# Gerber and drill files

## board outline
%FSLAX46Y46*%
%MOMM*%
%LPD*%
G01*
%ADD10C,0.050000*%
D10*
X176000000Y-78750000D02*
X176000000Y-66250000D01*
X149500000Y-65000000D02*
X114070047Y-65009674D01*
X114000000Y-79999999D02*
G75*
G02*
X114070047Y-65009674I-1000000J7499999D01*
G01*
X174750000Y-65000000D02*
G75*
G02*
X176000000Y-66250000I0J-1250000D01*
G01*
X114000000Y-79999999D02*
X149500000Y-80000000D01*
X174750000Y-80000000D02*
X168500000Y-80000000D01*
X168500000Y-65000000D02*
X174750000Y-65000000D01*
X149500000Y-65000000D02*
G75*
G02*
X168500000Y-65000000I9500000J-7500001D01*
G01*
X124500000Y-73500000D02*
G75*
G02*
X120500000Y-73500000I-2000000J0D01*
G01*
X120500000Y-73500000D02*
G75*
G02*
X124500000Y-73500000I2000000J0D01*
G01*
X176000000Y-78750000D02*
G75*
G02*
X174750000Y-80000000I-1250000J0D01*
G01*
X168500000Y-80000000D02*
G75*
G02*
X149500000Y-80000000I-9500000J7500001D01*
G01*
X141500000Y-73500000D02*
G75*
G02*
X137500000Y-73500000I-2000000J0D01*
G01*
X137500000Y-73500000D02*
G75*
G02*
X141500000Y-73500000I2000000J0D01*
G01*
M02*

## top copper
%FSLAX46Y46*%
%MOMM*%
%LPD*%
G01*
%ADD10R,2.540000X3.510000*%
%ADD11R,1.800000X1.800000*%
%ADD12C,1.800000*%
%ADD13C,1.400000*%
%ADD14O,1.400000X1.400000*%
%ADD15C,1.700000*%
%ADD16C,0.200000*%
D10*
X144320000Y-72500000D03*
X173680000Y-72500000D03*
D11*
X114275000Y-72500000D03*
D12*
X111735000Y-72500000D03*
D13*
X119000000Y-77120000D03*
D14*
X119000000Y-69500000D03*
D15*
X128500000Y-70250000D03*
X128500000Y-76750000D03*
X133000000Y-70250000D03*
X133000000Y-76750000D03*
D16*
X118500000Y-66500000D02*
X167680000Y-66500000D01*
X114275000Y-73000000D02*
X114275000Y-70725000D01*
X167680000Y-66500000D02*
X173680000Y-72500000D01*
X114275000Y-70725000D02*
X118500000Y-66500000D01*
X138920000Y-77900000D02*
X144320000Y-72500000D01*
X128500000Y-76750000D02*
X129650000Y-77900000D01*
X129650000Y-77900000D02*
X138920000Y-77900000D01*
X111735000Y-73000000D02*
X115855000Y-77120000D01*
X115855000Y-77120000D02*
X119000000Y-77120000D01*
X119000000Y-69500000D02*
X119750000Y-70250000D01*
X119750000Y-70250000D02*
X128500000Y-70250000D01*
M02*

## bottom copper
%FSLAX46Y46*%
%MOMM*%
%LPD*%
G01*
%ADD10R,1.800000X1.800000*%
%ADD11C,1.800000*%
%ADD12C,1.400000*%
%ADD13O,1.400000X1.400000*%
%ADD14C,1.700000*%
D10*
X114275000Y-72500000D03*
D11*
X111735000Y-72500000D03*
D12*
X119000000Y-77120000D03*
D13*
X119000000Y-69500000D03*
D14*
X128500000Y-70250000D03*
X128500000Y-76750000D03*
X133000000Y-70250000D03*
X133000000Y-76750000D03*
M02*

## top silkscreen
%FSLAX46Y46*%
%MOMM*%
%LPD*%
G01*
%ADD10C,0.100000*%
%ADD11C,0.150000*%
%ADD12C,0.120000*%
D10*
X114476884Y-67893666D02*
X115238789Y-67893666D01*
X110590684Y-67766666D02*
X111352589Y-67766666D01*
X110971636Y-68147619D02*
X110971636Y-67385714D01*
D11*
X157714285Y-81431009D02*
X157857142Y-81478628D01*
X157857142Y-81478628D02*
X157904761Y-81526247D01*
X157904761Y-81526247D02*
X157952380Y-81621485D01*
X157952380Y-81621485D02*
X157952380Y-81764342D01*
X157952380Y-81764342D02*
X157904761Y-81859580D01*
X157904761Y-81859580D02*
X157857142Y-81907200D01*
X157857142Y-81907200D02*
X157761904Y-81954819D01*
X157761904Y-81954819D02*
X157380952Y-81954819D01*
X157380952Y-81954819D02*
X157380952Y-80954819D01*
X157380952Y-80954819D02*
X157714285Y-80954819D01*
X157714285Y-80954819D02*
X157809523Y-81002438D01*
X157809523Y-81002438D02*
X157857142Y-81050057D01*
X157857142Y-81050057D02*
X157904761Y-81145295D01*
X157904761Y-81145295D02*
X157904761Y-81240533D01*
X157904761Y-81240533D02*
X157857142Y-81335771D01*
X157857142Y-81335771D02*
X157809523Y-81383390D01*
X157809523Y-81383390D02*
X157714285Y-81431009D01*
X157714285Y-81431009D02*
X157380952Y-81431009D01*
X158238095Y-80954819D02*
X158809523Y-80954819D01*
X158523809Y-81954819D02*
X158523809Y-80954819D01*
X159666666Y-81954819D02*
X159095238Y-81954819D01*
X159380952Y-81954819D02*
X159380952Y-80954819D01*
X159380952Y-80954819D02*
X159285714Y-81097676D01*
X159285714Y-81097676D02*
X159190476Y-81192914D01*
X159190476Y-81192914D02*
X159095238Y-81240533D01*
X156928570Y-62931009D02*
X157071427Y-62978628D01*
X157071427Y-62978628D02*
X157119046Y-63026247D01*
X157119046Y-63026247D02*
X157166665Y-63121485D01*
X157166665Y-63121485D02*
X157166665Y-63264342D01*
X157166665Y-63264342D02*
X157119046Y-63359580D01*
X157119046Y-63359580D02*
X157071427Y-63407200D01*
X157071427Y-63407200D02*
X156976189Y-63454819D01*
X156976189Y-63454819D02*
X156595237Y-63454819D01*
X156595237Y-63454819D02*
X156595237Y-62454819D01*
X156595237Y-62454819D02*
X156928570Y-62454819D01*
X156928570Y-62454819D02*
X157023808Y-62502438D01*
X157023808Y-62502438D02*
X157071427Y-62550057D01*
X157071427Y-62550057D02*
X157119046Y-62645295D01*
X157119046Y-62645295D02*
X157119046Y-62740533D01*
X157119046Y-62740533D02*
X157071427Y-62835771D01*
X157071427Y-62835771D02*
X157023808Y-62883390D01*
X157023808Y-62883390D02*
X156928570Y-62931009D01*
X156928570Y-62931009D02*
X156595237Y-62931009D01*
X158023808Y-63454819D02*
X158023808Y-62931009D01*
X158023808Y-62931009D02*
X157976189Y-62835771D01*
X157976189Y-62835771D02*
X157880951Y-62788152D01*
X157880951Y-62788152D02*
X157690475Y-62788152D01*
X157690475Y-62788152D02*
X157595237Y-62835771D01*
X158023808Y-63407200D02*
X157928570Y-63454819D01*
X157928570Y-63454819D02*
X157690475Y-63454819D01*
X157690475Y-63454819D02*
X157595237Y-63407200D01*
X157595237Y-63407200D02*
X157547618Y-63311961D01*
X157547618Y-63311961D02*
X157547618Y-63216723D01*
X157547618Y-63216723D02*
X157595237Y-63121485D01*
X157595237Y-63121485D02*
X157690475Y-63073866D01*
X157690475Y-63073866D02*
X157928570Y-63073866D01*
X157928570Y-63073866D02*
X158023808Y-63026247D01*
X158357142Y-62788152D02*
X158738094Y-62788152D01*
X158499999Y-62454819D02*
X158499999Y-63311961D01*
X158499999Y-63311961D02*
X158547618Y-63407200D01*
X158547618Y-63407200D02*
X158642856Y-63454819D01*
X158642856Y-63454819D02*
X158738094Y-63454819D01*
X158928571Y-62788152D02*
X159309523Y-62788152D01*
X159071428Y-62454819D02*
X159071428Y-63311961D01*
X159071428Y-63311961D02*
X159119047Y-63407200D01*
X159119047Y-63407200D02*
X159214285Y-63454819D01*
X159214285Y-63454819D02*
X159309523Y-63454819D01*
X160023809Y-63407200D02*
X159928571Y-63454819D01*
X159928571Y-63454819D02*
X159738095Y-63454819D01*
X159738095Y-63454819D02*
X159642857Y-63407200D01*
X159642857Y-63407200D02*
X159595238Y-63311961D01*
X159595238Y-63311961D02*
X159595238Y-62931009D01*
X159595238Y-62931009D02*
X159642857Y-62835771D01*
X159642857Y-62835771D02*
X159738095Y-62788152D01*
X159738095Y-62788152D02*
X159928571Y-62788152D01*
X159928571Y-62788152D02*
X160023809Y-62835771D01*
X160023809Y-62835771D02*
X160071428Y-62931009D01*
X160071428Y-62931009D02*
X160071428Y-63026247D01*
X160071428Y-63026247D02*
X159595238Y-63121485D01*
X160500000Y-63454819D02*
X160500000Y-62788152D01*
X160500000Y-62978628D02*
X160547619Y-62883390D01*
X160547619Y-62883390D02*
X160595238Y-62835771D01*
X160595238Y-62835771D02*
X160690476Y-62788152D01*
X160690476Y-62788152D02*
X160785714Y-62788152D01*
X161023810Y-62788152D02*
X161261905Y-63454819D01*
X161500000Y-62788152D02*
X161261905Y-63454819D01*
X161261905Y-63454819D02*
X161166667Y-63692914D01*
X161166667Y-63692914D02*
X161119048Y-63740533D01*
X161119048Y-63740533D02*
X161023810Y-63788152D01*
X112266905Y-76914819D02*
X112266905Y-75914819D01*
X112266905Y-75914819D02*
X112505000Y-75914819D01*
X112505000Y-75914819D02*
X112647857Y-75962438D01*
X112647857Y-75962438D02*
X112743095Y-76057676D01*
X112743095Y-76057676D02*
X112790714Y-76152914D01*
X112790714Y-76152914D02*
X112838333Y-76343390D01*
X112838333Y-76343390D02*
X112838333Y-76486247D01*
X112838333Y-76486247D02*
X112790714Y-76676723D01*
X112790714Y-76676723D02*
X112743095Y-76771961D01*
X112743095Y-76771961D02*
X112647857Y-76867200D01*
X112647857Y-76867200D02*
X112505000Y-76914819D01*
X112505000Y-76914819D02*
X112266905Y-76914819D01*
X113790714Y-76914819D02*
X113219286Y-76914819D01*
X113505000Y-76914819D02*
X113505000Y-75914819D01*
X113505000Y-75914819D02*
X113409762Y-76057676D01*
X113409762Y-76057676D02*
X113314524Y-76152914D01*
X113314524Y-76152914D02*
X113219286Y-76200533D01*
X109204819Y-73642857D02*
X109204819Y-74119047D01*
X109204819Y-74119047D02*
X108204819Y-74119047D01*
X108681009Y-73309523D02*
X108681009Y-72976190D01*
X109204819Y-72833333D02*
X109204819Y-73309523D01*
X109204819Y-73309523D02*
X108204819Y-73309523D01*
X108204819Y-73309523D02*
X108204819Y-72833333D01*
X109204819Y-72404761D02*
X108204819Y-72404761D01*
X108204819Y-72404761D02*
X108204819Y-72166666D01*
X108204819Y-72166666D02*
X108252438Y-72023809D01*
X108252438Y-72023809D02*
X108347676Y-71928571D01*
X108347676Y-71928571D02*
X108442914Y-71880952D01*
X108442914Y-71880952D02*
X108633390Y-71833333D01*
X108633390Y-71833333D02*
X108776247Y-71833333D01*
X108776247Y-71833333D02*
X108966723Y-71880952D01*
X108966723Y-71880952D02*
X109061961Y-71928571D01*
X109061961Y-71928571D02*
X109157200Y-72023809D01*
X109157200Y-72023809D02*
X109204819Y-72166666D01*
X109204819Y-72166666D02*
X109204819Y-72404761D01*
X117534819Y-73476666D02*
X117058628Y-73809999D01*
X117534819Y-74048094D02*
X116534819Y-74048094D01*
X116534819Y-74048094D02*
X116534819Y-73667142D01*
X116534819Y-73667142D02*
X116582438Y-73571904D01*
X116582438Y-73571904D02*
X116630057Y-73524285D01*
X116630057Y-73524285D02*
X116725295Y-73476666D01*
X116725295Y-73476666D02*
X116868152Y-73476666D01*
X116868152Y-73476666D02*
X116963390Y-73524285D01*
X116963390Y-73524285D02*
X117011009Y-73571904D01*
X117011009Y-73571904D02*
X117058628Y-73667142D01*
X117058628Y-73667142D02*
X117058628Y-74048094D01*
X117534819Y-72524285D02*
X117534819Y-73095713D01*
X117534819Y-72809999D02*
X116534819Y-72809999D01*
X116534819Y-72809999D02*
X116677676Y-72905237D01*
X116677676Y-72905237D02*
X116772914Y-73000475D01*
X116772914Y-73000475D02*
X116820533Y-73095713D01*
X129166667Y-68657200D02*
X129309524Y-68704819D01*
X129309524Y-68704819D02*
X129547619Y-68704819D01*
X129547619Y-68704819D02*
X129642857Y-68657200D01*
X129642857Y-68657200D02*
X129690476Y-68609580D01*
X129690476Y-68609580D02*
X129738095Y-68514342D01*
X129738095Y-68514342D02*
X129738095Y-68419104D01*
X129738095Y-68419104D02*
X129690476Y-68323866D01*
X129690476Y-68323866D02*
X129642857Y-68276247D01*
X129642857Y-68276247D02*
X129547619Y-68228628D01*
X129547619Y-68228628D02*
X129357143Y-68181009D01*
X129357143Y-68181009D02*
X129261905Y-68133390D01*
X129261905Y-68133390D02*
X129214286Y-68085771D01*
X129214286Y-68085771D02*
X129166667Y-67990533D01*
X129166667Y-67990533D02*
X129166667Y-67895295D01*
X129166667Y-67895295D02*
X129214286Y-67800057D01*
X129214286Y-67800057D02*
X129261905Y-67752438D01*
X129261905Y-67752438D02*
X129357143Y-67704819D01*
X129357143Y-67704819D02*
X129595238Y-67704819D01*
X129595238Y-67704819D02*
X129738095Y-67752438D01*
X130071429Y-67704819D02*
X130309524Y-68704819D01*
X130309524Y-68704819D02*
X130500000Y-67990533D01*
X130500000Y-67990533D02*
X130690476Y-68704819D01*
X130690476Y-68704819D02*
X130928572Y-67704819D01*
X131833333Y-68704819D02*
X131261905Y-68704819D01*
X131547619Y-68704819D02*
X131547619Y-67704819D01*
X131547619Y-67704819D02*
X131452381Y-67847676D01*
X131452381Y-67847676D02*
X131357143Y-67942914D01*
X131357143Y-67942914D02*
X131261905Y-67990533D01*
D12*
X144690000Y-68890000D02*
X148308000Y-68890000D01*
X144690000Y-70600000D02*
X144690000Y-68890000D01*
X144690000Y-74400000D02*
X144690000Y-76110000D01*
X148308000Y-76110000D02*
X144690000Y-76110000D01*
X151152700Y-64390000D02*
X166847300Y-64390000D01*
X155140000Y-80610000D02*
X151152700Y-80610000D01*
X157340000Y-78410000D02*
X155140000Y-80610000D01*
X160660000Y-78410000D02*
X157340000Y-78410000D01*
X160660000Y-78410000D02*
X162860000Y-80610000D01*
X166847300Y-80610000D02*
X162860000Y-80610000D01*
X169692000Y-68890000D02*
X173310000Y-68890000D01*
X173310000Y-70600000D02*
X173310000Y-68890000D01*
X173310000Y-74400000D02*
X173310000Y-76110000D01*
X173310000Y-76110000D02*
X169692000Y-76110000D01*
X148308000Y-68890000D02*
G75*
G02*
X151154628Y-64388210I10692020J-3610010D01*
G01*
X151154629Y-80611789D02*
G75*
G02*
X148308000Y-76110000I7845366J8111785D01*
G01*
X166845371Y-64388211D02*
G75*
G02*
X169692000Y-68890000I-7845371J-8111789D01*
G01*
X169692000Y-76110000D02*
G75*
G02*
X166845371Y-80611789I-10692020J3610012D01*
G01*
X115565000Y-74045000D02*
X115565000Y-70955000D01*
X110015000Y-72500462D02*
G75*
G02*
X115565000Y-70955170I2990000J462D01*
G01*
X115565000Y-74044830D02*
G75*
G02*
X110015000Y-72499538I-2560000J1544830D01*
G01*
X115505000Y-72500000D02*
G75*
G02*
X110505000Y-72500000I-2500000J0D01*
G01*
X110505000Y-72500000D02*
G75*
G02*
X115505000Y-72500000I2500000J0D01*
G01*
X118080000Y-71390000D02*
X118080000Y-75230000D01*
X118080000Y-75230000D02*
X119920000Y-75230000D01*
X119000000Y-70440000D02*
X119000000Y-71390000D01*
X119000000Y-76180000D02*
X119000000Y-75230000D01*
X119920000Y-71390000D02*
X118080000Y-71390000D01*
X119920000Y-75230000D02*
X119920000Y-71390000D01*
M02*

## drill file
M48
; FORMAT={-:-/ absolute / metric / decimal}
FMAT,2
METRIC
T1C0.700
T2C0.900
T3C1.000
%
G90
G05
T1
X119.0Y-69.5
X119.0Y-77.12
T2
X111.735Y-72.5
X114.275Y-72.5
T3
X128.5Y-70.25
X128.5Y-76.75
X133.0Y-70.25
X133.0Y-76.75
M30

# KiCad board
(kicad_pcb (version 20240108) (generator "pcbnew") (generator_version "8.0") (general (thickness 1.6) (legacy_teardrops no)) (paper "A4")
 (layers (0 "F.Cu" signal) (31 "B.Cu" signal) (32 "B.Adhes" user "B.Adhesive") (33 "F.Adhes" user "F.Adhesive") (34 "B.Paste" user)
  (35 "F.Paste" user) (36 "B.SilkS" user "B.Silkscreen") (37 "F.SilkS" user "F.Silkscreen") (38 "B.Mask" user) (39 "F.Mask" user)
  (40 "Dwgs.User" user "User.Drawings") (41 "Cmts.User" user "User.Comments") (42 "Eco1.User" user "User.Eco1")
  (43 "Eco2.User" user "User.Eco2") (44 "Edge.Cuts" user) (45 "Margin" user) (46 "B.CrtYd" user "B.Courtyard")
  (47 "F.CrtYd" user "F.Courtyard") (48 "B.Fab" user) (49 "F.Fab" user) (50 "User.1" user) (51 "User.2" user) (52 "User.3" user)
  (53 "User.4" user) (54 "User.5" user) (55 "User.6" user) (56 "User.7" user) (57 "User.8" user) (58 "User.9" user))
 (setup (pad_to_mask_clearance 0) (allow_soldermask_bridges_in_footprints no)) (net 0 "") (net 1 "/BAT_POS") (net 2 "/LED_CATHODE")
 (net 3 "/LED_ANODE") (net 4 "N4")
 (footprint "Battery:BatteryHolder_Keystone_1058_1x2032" (layer "F.Cu") (at 159 72.5)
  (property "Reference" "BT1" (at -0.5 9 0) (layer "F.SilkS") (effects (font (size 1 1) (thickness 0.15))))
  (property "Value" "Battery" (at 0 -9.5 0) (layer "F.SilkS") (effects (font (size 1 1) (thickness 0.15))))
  (fp_line (start -14.31 -3.61) (end -10.692 -3.61) (stroke (width 0.12) (type solid)) (layer "F.SilkS"))
  (fp_line (start -14.31 -1.9) (end -14.31 -3.61) (stroke (width 0.12) (type solid)) (layer "F.SilkS"))
  (fp_line (start -14.31 1.9) (end -14.31 3.61) (stroke (width 0.12) (type solid)) (layer "F.SilkS"))
  (fp_line (start -10.692 3.61) (end -14.31 3.61) (stroke (width 0.12) (type solid)) (layer "F.SilkS"))
  (fp_line (start -7.8473 -8.11) (end 7.8473 -8.11) (stroke (width 0.12) (type solid)) (layer "F.SilkS"))
  (fp_line (start -3.86 8.11) (end -7.8473 8.11) (stroke (width 0.12) (type solid)) (layer "F.SilkS"))
  (fp_line (start -1.66 5.91) (end -3.86 8.11) (stroke (width 0.12) (type solid)) (layer "F.SilkS"))
  (fp_line (start 1.66 5.91) (end -1.66 5.91) (stroke (width 0.12) (type solid)) (layer "F.SilkS"))
  (fp_line (start 1.66 5.91) (end 3.86 8.11) (stroke (width 0.12) (type solid)) (layer "F.SilkS"))
  (fp_line (start 7.8473 8.11) (end 3.86 8.11) (stroke (width 0.12) (type solid)) (layer "F.SilkS"))
  (fp_line (start 10.692 -3.61) (end 14.31 -3.61) (stroke (width 0.12) (type solid)) (layer "F.SilkS"))
  (fp_line (start 14.31 -1.9) (end 14.31 -3.61) (stroke (width 0.12) (type solid)) (layer "F.SilkS"))
  (fp_line (start 14.31 1.9) (end 14.31 3.61) (stroke (width 0.12) (type solid)) (layer "F.SilkS"))
  (fp_line (start 14.31 3.61) (end 10.692 3.61) (stroke (width 0.12) (type solid)) (layer "F.SilkS"))
  (fp_arc (start -10.692 -3.61) (mid -9.538084 -6.031244) (end -7.845371 -8.111789) (stroke (width 0.12) (type solid)) (layer "F.SilkS"))
  (fp_arc (start -7.845371 8.111789) (mid -9.538085 6.031244) (end -10.692 3.61) (stroke (width 0.12) (type solid)) (layer "F.SilkS"))
  (fp_arc (start 7.845371 -8.111789) (mid 9.538085 -6.031244) (end 10.692 -3.61) (stroke (width 0.12) (type solid)) (layer "F.SilkS"))
  (fp_arc (start 10.692 3.61) (mid 9.538084 6.031244) (end 7.845371 8.111789) (stroke (width 0.12) (type solid)) (layer "F.SilkS"))
  (pad "1" smd rect (at -14.68 0) (size 2.54 3.51) (layers "F.Cu" "F.Paste" "F.Mask") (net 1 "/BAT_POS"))
  (pad "2" smd rect (at 14.68 0) (size 2.54 3.51) (layers "F.Cu" "F.Paste" "F.Mask") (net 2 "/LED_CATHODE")))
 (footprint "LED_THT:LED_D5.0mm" (layer "F.Cu") (at 114.275 72.5 180)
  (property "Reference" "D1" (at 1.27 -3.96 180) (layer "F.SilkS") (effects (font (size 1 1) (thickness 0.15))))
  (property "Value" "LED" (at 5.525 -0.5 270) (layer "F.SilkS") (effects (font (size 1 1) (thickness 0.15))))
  (fp_line (start -1.29 -1.545) (end -1.29 1.545) (stroke (width 0.12) (type solid)) (layer "F.SilkS"))
  (fp_arc (start 4.26 -0.000462) (mid 2.072002 2.880433) (end -1.29 1.54483) (stroke (width 0.12) (type solid)) (layer "F.SilkS"))
  (fp_arc (start -1.29 -1.54483) (mid 2.072002 -2.880433) (end 4.26 0.000462) (stroke (width 0.12) (type solid)) (layer "F.SilkS"))
  (fp_circle (center 1.27 0) (end 3.77 0) (stroke (width 0.12) (type solid)) (fill none) (layer "F.SilkS"))
  (pad "1" thru_hole rect (at 0 0 180) (size 1.8 1.8) (drill 0.9) (layers "*.Cu" "*.Mask") (remove_unused_layers no) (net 2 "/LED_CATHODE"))
  (pad "2" thru_hole circle (at 2.54 0 180) (size 1.8 1.8) (drill 0.9) (layers "*.Cu" "*.Mask") (remove_unused_layers no)
   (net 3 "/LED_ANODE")))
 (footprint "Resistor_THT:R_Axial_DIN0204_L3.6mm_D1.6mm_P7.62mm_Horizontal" (layer "F.Cu") (at 119 77.12 90)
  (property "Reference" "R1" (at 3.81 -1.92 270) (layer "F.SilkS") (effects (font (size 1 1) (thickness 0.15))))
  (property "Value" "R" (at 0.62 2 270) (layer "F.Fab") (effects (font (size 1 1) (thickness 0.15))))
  (fp_line (start 5.73 -0.92) (end 1.89 -0.92) (stroke (width 0.12) (type solid)) (layer "F.SilkS"))
  (fp_line (start 1.89 -0.92) (end 1.89 0.92) (stroke (width 0.12) (type solid)) (layer "F.SilkS"))
  (fp_line (start 6.68 0) (end 5.73 0) (stroke (width 0.12) (type solid)) (layer "F.SilkS"))
  (fp_line (start 0.94 0) (end 1.89 0) (stroke (width 0.12) (type solid)) (layer "F.SilkS"))
  (fp_line (start 5.73 0.92) (end 5.73 -0.92) (stroke (width 0.12) (type solid)) (layer "F.SilkS"))
  (fp_line (start 1.89 0.92) (end 5.73 0.92) (stroke (width 0.12) (type solid)) (layer "F.SilkS"))
  (pad "1" thru_hole circle (at 0 0 90) (size 1.4 1.4) (drill 0.7) (layers "*.Cu" "*.Mask") (remove_unused_layers no) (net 3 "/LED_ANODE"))
  (pad "2" thru_hole oval (at 7.62 0 90) (size 1.4 1.4) (drill 0.7) (layers "*.Cu" "*.Mask") (remove_unused_layers no) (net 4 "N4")))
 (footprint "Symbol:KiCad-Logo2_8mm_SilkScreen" (layer "B.Cu") (at 159.259893 72.176424 180)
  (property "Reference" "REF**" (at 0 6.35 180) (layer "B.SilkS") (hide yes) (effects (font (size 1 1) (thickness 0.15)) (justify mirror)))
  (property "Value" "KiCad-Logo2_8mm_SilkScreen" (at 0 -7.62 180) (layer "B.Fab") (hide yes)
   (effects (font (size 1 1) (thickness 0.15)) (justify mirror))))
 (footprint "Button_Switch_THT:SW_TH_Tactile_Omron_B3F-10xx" (layer "B.Cu") (at 128.5 70.25 -90)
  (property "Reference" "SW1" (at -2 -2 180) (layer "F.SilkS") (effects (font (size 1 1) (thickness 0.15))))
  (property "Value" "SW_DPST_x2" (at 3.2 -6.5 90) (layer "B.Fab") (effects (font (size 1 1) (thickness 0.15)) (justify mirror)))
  (pad "1" thru_hole circle (at 0 0 270) (size 1.7 1.7) (drill 1) (layers "*.Cu" "*.Mask") (remove_unused_layers no) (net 4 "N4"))
  (pad "2" thru_hole circle (at 6.5 0 270) (size 1.7 1.7) (drill 1) (layers "*.Cu" "*.Mask") (remove_unused_layers no) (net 1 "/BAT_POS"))
  (pad "3" thru_hole circle (at 0 -4.5 270) (size 1.7 1.7) (drill 1) (layers "*.Cu" "*.Mask") (remove_unused_layers no))
  (pad "4" thru_hole circle (at 6.5 -4.5 270) (size 1.7 1.7) (drill 1) (layers "*.Cu" "*.Mask") (remove_unused_layers no)))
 (gr_line (start 176 78.75) (end 176 66.25) (stroke (width 0.05) (type default)) (layer "Edge.Cuts"))
 (gr_line (start 149.5 65) (end 114.070047 65.009674) (stroke (width 0.05) (type default)) (layer "Edge.Cuts"))
 (gr_arc (start 114 79.999999) (mid 105.433711 72.464644) (end 114.070047 65.009674) (stroke (width 0.05) (type default))
  (layer "Edge.Cuts"))
 (gr_arc (start 174.75 65) (mid 175.633883 65.366117) (end 176 66.25) (stroke (width 0.05) (type default)) (layer "Edge.Cuts"))
 (gr_line (start 114 79.999999) (end 149.5 80) (stroke (width 0.05) (type default)) (layer "Edge.Cuts"))
 (gr_line (start 174.75 80) (end 168.5 80) (stroke (width 0.05) (type default)) (layer "Edge.Cuts"))
 (gr_line (start 168.5 65) (end 174.75 65) (stroke (width 0.05) (type default)) (layer "Edge.Cuts"))
 (gr_arc (start 149.5 65) (mid 159 60.396282) (end 168.5 65) (stroke (width 0.05) (type default)) (layer "Edge.Cuts"))
 (gr_circle (center 122.5 73.5) (end 124.5 73.5) (stroke (width 0.05) (type default)) (fill none) (layer "Edge.Cuts"))
 (gr_arc (start 176 78.75) (mid 175.633883 79.633883) (end 174.75 80) (stroke (width 0.05) (type default)) (layer "Edge.Cuts"))
 (gr_arc (start 168.5 80) (mid 159 84.603718) (end 149.5 80) (stroke (width 0.05) (type default)) (layer "Edge.Cuts"))
 (gr_circle (center 139.5 73.5) (end 141.5 73.5) (stroke (width 0.05) (type default)) (fill none) (layer "Edge.Cuts"))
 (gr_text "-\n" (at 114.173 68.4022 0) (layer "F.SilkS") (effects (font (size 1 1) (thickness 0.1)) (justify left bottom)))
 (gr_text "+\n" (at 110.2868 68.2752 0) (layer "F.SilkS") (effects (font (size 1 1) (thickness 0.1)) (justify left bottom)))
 (segment (start 118.5 66.5) (end 167.68 66.5) (width 0.2) (layer "F.Cu") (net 2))
 (segment (start 114.275 73) (end 114.275 70.725) (width 0.2) (layer "F.Cu") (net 2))
 (segment (start 167.68 66.5) (end 173.68 72.5) (width 0.2) (layer "F.Cu") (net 2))
 (segment (start 114.275 70.725) (end 118.5 66.5) (width 0.2) (layer "F.Cu") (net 2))
 (segment (start 138.92 77.9) (end 144.32 72.5) (width 0.2) (layer "F.Cu") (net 1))
 (segment (start 128.5 76.75) (end 129.65 77.9) (width 0.2) (layer "F.Cu") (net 1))
 (segment (start 129.65 77.9) (end 138.92 77.9) (width 0.2) (layer "F.Cu") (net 1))
 (segment (start 111.735 73) (end 115.855 77.12) (width 0.2) (layer "F.Cu") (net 3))
 (segment (start 115.855 77.12) (end 119 77.12) (width 0.2) (layer "F.Cu") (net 3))
 (segment (start 119 69.5) (end 119.75 70.25) (width 0.2) (layer "F.Cu") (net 4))
 (segment (start 119.75 70.25) (end 128.5 70.25) (width 0.2) (layer "F.Cu") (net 4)))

